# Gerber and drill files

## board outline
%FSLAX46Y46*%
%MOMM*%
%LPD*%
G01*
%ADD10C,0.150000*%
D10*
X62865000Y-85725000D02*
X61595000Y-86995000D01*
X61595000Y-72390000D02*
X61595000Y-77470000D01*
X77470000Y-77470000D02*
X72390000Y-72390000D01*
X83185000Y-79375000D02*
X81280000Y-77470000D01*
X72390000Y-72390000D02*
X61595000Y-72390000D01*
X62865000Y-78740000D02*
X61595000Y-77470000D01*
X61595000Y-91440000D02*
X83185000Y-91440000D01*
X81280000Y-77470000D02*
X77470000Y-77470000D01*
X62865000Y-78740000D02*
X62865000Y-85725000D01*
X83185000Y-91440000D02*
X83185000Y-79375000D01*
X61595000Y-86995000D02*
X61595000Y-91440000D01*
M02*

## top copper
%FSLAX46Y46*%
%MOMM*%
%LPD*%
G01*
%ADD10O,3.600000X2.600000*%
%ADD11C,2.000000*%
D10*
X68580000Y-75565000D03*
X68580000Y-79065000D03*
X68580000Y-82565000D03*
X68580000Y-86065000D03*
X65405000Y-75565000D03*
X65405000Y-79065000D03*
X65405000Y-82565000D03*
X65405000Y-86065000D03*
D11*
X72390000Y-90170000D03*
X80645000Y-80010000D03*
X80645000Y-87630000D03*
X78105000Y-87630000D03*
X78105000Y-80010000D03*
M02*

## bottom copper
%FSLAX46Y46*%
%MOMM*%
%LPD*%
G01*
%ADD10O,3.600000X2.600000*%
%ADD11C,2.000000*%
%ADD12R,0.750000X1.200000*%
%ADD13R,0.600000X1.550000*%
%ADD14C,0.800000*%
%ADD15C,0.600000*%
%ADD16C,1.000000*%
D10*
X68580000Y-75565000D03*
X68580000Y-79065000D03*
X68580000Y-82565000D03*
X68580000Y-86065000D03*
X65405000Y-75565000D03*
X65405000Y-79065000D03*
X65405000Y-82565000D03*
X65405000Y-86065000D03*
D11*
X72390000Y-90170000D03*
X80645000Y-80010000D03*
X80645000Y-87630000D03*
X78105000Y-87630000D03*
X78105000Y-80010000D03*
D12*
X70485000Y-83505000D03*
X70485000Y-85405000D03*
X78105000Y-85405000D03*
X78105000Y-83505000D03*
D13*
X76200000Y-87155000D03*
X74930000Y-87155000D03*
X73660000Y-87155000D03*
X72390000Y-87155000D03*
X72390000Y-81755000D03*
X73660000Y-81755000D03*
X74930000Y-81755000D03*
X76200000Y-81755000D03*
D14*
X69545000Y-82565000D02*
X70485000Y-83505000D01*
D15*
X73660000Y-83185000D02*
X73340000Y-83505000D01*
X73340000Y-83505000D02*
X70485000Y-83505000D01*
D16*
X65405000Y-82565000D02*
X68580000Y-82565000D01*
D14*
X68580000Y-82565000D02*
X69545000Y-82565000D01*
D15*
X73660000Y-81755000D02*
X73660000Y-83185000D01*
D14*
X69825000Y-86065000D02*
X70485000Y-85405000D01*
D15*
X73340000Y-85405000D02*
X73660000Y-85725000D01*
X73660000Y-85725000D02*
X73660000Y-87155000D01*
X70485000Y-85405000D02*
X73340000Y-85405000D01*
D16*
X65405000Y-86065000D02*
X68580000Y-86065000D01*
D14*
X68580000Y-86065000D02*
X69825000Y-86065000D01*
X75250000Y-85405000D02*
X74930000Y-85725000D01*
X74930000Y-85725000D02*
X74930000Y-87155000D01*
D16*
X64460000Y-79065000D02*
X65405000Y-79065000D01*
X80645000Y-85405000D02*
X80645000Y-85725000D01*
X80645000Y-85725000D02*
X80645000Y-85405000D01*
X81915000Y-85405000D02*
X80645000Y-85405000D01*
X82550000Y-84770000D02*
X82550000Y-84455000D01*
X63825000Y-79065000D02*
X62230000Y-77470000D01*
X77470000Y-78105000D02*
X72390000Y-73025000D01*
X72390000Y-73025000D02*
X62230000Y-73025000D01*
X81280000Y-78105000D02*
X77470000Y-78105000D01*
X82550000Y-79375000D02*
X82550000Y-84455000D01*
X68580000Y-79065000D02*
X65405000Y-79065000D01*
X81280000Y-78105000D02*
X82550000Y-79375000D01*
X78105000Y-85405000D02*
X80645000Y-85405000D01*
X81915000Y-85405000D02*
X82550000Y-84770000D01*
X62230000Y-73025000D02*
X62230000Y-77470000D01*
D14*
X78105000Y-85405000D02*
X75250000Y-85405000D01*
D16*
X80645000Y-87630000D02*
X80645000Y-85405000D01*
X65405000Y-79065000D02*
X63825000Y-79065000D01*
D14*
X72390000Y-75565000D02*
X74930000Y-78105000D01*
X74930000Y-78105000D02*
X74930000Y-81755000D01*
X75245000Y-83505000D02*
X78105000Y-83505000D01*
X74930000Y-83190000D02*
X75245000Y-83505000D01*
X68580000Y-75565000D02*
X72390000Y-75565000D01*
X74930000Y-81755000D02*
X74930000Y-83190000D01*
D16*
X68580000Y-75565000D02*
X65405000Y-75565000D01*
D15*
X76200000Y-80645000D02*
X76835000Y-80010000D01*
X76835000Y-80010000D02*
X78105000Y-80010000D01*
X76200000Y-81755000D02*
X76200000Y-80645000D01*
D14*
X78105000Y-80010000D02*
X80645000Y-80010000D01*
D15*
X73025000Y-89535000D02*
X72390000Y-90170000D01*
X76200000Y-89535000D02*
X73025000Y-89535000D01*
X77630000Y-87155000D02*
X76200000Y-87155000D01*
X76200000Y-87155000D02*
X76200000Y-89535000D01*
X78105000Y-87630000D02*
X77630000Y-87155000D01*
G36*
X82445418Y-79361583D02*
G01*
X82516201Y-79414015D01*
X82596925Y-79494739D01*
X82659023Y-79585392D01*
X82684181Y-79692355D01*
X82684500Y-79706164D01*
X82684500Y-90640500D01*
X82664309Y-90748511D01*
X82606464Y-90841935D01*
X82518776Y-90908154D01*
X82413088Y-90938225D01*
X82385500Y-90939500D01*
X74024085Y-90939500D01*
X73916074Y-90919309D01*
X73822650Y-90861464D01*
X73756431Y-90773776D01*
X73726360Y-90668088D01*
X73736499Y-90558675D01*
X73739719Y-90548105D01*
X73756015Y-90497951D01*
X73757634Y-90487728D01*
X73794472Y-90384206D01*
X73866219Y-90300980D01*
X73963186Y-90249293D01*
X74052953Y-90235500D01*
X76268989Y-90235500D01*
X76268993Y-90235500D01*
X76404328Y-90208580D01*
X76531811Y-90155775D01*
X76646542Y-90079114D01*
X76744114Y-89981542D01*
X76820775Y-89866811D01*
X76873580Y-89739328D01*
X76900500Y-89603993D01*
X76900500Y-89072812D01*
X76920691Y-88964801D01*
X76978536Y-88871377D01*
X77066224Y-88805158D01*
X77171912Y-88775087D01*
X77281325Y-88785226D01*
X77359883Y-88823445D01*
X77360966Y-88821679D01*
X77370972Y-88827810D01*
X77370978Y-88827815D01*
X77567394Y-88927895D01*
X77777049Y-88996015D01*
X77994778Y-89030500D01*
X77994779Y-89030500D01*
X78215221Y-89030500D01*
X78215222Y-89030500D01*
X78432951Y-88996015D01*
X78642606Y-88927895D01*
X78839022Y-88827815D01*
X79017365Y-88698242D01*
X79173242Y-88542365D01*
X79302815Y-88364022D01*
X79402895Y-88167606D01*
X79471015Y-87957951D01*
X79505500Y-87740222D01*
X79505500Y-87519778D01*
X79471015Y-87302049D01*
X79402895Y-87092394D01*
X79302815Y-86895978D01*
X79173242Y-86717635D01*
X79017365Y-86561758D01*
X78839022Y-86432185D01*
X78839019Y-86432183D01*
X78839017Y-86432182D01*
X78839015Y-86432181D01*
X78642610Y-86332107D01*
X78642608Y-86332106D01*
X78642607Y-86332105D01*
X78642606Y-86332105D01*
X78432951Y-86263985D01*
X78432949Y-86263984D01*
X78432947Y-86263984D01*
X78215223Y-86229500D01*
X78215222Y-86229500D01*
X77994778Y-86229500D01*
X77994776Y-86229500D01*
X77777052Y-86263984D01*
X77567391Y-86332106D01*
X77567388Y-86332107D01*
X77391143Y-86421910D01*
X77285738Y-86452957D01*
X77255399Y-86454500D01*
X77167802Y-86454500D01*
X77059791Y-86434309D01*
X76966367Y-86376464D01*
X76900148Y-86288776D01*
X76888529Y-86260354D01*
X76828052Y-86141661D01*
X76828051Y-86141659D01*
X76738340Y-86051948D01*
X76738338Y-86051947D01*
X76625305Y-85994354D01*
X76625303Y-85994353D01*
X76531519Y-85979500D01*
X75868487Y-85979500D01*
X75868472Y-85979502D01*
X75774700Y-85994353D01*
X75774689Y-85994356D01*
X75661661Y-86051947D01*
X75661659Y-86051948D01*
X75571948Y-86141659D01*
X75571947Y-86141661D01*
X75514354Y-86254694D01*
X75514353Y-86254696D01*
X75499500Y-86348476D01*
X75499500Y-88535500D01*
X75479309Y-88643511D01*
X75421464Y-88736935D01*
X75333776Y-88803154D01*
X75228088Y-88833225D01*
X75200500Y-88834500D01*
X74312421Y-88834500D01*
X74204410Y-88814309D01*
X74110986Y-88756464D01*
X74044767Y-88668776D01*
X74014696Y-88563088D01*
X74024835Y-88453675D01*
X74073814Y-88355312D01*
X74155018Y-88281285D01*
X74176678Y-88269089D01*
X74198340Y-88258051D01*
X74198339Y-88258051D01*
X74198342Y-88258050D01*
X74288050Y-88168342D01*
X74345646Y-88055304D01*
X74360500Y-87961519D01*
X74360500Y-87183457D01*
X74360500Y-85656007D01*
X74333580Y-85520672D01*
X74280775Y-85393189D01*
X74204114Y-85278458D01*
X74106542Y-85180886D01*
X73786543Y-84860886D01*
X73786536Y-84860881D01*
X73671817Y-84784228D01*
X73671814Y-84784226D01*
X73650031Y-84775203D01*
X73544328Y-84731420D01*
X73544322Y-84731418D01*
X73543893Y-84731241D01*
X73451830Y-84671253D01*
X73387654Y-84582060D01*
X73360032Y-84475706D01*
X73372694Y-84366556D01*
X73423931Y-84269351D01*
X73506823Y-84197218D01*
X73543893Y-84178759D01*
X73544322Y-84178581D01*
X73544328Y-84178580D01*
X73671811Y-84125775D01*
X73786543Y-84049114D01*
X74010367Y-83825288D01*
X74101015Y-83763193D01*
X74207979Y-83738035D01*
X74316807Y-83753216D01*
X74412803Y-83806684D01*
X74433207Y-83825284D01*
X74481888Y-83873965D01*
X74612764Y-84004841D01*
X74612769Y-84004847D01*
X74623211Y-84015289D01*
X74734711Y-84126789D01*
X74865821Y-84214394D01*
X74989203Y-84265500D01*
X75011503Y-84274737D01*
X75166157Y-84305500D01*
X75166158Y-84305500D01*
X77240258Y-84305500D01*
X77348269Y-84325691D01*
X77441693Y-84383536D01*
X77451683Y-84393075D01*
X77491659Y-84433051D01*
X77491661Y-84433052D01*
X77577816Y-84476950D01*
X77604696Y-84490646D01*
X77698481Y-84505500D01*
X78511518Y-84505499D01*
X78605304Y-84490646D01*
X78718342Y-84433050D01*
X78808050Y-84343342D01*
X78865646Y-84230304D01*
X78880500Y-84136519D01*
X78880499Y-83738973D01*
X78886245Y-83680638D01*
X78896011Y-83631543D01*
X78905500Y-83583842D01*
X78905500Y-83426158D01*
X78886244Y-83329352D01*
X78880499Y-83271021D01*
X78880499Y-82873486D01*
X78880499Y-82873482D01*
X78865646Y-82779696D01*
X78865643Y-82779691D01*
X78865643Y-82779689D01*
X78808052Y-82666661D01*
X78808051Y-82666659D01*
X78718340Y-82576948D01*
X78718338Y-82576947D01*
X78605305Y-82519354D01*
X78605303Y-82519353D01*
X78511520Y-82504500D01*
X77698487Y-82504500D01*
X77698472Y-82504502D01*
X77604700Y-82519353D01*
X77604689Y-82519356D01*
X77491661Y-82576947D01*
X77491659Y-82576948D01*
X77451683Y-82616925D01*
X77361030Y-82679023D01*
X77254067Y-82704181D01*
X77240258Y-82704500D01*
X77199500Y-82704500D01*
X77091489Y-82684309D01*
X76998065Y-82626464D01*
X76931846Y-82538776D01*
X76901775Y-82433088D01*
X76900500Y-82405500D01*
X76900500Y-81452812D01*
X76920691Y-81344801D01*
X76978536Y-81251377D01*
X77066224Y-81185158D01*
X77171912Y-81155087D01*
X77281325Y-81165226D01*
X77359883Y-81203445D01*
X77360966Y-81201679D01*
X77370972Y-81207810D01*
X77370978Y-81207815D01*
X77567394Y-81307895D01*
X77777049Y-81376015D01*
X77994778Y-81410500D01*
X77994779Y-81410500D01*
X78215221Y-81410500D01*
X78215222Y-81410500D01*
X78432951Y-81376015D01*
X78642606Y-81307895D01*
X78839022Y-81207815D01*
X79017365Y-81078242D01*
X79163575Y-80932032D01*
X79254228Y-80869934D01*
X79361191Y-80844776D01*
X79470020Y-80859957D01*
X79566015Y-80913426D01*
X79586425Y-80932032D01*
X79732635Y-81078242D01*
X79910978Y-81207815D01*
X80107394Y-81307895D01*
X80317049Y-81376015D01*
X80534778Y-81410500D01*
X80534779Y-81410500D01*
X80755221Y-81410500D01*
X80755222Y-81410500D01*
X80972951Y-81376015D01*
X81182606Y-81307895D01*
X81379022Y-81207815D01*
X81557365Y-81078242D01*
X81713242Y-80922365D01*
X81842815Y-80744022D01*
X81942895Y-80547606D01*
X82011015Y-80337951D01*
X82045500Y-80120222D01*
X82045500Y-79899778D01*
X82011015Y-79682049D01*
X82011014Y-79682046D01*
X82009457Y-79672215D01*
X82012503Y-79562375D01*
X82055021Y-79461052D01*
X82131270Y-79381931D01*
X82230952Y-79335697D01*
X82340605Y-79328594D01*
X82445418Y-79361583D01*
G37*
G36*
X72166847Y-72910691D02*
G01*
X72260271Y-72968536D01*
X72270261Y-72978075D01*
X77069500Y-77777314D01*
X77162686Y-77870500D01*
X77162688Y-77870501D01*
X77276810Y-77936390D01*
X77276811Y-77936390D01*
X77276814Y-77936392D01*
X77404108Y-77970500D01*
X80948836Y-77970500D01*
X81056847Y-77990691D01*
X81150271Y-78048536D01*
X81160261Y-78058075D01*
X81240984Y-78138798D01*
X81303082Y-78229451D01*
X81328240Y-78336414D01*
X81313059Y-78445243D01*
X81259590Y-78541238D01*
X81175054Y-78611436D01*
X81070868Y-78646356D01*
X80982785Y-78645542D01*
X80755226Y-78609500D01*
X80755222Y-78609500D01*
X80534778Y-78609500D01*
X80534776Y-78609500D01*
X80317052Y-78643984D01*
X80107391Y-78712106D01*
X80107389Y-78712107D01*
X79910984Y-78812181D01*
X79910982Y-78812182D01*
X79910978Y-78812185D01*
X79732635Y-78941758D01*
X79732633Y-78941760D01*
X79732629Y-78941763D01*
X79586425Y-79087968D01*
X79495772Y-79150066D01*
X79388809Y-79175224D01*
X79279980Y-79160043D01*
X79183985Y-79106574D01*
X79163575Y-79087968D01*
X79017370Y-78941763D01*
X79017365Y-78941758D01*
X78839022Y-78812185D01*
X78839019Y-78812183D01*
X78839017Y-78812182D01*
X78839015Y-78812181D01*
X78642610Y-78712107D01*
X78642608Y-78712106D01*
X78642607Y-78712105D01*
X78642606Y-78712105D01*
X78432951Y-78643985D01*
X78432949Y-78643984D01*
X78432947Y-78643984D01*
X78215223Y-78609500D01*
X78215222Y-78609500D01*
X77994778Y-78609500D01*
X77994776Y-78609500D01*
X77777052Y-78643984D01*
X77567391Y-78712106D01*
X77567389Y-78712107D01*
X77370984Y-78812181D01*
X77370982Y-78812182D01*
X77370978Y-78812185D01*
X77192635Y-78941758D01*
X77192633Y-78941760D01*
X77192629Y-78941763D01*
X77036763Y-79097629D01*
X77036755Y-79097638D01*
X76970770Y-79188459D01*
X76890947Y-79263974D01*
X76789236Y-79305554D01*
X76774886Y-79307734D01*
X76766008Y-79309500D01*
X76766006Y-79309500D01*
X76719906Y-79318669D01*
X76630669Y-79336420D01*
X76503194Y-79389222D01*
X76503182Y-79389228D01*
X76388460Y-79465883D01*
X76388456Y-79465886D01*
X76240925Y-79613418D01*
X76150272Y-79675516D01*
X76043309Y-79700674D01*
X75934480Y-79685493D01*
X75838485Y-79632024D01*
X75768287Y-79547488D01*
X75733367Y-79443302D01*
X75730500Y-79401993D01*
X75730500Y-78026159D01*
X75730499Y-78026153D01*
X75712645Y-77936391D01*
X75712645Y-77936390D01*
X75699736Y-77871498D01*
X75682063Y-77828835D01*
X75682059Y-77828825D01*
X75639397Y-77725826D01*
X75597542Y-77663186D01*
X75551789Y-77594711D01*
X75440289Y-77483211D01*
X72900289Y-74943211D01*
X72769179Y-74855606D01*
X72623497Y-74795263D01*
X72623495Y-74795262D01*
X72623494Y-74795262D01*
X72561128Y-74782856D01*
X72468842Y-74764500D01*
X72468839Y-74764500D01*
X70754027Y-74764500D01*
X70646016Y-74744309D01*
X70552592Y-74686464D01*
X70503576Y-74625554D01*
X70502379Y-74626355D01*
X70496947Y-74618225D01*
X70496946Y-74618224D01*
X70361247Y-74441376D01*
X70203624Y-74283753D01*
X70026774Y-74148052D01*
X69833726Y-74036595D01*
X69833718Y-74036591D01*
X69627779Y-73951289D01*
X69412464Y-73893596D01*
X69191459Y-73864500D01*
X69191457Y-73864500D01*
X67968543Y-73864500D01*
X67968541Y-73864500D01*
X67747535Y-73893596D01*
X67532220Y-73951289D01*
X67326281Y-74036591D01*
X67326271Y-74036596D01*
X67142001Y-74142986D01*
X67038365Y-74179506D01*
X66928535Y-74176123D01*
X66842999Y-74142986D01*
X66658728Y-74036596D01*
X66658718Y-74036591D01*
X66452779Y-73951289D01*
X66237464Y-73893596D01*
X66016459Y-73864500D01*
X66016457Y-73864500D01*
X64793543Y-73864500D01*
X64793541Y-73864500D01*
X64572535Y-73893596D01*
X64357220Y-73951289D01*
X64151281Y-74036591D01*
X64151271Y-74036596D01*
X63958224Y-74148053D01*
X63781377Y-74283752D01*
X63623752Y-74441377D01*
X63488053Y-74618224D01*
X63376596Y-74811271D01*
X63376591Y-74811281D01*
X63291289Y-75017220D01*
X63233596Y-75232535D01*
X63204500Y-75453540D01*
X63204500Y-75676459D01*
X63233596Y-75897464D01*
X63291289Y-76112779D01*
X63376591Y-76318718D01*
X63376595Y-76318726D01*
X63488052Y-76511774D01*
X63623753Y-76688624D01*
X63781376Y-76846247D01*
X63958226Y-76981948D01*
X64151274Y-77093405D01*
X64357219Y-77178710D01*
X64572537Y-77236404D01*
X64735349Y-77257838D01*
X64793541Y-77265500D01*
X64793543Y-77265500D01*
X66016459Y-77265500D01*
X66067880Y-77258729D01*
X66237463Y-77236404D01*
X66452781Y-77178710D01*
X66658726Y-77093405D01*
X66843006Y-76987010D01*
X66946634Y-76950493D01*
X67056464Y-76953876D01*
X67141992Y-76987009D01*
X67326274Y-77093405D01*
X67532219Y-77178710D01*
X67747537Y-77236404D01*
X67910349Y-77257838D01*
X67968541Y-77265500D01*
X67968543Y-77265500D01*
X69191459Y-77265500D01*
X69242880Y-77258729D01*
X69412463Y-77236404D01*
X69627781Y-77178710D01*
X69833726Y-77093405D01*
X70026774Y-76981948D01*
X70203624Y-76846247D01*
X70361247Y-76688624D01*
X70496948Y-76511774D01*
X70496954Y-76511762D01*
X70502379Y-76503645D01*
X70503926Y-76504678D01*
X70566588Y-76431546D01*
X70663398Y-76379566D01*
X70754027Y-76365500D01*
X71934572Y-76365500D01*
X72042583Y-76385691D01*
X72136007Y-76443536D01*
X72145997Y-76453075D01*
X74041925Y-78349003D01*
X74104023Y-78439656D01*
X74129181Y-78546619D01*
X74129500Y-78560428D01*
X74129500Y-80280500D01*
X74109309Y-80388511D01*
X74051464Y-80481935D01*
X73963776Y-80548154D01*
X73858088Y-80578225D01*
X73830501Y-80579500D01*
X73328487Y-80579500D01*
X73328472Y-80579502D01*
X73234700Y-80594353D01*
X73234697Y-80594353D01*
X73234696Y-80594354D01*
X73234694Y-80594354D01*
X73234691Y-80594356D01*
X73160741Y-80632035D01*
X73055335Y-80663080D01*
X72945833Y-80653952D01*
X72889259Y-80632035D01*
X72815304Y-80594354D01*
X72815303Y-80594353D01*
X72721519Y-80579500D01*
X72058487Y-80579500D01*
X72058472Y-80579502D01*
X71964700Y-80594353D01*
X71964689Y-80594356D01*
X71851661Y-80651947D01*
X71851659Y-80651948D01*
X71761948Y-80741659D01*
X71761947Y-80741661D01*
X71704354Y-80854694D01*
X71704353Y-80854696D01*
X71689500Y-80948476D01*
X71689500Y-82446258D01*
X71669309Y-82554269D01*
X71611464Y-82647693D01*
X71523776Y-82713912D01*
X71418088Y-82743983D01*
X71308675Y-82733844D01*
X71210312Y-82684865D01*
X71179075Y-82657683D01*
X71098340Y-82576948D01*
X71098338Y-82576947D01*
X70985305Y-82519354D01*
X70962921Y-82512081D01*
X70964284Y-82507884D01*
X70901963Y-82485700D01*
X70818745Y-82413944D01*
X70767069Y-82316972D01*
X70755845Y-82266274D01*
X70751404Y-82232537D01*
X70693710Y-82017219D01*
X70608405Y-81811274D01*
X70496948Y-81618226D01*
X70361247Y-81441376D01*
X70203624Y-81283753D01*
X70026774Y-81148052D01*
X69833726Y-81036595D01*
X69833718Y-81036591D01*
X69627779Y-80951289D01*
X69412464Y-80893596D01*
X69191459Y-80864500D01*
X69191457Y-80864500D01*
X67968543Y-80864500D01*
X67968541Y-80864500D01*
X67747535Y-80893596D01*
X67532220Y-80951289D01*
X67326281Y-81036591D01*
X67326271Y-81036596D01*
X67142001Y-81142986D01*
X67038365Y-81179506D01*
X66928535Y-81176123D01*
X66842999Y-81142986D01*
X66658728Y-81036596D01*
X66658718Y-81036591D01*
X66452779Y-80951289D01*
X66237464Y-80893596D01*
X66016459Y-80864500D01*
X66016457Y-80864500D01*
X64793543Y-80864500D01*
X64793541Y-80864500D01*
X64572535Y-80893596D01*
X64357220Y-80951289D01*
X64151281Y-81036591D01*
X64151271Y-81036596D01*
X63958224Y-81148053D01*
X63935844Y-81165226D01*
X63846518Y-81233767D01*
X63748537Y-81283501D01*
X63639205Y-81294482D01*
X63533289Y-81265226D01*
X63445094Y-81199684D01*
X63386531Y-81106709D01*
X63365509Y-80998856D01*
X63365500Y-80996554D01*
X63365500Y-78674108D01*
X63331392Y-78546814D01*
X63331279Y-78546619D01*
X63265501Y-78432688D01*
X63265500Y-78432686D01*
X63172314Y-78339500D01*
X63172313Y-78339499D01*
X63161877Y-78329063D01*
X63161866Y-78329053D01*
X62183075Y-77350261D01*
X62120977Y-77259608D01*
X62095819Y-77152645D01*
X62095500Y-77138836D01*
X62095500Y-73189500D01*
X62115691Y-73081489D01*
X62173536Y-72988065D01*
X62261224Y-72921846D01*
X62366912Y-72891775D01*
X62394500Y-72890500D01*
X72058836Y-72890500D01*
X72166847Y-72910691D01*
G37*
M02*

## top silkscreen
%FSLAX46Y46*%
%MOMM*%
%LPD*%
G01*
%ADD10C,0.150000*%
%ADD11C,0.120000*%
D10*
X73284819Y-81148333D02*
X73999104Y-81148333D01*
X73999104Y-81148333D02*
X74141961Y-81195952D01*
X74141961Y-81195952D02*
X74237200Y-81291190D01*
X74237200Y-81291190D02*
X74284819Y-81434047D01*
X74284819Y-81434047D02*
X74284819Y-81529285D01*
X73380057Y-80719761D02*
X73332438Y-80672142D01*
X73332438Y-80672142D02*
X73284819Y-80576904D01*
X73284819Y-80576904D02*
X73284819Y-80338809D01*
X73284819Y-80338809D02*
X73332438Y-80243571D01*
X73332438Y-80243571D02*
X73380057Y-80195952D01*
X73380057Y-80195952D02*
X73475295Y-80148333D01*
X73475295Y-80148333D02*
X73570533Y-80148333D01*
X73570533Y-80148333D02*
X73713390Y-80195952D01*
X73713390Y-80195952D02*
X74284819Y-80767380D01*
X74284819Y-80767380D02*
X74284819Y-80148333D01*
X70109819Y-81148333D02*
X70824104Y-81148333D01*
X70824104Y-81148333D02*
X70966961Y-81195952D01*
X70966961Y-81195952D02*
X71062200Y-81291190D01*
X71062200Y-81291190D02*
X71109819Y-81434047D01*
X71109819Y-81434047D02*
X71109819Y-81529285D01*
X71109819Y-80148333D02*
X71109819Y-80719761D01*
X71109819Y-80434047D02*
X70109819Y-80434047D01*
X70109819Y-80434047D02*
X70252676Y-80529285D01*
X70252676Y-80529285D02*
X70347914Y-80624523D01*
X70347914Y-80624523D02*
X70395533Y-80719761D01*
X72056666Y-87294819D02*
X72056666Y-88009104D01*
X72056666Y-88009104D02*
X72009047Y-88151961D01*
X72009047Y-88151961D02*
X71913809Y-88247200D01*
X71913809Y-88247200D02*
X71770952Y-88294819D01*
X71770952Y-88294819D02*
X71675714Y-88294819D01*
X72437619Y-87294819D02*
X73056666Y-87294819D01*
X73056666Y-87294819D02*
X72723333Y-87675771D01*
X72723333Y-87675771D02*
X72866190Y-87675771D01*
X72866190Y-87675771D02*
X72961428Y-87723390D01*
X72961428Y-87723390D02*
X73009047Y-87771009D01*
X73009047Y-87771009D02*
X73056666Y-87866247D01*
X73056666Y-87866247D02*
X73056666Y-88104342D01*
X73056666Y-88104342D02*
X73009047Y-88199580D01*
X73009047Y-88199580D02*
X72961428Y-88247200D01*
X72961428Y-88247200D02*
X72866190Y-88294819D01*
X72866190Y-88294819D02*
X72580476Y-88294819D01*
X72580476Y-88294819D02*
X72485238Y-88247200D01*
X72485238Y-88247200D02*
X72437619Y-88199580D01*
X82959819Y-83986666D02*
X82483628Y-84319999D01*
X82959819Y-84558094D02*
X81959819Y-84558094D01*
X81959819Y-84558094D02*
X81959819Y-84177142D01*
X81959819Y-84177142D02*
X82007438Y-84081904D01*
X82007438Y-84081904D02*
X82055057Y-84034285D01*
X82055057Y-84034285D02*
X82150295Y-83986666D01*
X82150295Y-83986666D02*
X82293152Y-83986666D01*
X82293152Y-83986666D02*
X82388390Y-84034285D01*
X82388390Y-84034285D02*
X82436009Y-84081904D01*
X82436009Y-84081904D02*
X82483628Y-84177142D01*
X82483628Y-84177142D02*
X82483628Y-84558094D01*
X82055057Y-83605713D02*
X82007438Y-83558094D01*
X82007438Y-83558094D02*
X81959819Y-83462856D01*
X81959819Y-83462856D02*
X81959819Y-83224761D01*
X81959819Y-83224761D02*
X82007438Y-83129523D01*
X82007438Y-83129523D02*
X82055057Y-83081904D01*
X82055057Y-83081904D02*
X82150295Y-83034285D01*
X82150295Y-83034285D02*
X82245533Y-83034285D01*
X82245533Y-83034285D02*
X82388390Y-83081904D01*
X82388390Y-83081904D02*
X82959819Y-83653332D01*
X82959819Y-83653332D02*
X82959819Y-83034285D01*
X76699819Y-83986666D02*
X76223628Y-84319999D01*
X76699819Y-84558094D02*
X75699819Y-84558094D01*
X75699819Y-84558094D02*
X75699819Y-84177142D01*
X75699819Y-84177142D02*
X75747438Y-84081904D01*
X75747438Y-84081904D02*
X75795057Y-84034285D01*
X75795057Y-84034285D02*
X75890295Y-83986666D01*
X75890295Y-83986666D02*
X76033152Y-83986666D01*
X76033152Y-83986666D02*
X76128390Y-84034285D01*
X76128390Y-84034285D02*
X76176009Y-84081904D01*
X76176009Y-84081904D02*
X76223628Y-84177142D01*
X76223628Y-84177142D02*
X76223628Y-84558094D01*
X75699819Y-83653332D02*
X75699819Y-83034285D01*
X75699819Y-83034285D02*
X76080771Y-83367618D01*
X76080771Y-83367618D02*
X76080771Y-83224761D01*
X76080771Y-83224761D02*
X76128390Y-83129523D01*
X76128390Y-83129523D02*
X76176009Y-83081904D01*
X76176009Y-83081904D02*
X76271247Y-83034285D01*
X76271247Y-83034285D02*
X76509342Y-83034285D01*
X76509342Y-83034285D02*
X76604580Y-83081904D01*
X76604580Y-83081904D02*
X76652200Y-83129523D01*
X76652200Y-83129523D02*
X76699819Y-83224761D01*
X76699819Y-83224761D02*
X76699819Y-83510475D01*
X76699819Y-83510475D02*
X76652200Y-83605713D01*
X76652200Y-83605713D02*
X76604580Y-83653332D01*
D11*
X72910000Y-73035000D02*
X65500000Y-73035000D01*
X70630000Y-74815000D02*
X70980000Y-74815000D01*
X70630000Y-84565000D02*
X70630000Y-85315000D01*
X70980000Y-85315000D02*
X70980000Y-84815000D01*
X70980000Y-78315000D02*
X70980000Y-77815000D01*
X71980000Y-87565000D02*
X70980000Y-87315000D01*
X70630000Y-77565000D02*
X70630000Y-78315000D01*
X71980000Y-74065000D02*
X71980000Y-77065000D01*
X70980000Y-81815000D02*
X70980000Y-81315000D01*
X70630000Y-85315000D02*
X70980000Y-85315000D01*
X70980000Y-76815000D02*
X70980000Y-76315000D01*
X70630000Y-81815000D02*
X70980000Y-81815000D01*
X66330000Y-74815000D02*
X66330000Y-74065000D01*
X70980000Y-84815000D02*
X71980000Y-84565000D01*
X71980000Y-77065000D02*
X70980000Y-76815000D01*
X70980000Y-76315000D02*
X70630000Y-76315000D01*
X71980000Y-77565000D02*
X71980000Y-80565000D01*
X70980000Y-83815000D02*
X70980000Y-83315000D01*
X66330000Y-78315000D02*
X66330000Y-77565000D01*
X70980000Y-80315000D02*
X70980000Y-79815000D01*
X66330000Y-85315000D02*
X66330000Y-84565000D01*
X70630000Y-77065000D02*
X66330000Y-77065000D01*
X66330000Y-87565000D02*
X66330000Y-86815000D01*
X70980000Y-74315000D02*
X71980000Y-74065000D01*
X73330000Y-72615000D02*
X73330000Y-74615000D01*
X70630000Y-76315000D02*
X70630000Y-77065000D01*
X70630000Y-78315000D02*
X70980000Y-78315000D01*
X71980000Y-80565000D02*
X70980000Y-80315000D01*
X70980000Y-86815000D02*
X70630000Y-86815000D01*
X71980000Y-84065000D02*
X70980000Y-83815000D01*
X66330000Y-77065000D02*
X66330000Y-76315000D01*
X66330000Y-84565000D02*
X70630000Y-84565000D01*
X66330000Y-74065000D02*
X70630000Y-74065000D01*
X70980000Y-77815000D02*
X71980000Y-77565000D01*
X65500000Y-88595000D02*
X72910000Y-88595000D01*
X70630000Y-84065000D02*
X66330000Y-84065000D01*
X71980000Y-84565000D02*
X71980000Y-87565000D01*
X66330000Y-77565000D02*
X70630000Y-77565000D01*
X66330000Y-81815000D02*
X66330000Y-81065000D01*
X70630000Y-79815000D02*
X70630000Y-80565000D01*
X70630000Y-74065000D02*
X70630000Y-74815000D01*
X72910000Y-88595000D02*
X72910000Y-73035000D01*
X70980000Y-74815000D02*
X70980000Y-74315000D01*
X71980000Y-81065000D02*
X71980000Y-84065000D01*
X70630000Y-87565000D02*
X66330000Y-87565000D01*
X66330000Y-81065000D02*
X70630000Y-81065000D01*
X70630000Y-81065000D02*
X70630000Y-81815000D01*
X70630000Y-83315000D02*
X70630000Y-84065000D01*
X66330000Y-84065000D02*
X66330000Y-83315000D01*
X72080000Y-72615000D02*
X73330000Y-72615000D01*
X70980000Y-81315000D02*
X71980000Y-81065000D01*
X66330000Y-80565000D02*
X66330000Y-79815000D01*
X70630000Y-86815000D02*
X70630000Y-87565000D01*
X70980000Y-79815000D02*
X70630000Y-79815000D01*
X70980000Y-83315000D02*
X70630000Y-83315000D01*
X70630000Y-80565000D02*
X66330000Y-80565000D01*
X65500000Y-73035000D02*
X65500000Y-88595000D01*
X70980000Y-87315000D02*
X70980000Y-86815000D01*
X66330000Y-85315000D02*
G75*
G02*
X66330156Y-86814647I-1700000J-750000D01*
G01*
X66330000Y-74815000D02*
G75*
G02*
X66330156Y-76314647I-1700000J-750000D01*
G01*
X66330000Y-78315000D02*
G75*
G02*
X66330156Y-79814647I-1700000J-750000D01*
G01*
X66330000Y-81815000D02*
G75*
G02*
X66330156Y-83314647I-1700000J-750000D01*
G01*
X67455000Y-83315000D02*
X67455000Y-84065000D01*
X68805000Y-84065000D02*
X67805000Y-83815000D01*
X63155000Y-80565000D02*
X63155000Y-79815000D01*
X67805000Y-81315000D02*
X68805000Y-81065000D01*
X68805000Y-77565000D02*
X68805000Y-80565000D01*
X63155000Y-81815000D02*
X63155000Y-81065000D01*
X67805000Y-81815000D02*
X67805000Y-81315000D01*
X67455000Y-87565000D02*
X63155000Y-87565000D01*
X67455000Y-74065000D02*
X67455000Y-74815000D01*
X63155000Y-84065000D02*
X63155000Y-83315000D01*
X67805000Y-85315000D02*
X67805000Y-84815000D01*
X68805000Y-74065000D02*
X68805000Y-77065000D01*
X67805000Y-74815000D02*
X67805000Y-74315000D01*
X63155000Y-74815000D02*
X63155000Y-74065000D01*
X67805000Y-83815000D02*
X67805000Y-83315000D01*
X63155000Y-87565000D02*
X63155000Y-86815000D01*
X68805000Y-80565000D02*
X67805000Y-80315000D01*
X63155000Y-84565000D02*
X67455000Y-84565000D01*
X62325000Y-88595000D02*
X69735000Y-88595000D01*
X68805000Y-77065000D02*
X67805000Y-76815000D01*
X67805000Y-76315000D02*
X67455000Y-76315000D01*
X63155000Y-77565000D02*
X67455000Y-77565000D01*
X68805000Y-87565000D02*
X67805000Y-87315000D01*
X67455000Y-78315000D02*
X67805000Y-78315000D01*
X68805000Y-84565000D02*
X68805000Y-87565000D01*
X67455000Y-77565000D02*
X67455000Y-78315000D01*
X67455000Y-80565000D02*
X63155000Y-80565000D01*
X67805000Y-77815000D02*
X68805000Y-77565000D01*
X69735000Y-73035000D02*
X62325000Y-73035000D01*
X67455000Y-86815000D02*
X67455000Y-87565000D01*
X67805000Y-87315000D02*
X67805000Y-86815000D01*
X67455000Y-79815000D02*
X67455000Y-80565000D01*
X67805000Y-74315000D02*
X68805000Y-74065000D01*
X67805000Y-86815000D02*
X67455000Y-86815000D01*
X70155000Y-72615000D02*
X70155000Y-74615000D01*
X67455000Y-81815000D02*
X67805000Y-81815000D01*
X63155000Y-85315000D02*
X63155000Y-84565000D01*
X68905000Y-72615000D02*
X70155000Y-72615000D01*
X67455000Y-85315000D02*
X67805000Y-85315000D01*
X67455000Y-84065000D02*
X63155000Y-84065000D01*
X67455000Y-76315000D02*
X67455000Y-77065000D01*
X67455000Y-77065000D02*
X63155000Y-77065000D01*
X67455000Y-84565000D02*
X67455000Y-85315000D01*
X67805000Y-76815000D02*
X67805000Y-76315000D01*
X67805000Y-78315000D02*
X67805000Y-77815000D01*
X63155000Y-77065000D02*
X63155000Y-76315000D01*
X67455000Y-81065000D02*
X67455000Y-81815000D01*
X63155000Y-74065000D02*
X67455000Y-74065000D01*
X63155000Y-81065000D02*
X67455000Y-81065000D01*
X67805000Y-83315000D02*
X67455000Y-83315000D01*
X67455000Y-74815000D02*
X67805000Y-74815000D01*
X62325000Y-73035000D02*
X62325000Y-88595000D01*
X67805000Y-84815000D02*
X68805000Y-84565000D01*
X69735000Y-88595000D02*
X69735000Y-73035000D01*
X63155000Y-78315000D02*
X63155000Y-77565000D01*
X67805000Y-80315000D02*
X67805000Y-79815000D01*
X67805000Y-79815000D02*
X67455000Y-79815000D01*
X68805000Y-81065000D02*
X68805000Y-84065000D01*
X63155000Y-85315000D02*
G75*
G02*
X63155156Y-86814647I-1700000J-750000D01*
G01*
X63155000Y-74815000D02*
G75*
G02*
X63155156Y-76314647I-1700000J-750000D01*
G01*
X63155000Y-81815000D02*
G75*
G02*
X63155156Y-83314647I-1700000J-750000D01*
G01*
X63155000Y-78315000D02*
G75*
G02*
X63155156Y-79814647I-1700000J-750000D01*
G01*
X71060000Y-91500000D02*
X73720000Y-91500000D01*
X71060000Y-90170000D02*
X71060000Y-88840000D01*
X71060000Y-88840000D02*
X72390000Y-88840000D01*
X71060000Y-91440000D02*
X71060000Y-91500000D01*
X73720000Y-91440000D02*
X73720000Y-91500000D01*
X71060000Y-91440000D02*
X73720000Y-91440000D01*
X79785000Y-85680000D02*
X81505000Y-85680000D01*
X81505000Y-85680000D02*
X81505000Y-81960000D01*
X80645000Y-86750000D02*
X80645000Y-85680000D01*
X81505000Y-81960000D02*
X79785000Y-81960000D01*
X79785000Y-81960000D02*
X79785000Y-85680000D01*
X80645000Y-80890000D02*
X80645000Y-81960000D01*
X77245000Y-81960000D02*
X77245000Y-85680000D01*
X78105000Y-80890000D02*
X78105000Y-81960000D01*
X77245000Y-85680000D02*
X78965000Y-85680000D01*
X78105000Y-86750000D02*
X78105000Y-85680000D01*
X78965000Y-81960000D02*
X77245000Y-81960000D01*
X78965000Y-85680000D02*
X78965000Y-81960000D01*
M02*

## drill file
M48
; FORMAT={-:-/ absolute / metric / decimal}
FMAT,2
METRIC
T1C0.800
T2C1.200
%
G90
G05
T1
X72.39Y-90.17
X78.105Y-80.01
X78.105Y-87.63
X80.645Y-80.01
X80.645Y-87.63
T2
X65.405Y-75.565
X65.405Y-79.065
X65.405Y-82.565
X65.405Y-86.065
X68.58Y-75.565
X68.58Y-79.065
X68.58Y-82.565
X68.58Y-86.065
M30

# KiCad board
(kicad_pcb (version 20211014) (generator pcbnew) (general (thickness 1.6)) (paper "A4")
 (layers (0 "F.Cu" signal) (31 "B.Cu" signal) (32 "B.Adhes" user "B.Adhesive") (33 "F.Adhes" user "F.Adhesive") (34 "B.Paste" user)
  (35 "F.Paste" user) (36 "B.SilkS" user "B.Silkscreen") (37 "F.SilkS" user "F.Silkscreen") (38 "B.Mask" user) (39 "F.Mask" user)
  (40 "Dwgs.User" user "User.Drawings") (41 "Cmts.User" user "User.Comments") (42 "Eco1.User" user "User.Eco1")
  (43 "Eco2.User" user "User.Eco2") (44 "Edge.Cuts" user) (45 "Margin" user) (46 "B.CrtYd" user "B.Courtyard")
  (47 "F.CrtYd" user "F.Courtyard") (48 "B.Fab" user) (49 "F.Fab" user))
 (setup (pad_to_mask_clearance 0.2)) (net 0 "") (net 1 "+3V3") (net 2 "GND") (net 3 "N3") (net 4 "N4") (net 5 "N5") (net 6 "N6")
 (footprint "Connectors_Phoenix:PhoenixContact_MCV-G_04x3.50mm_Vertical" (layer "F.Cu") (at 68.58 75.565 -90)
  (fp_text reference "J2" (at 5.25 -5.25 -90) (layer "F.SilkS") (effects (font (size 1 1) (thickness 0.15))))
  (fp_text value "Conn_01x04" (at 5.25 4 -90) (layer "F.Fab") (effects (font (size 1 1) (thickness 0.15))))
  (fp_line (start -2.53 -4.33) (end -2.53 3.08) (layer "F.SilkS") (width 0.12))
  (fp_line (start -0.75 -2.05) (end -0.75 -2.4) (layer "F.SilkS") (width 0.12))
  (fp_line (start 9 -2.05) (end 9.75 -2.05) (layer "F.SilkS") (width 0.12))
  (fp_line (start 9.75 -2.4) (end 9.25 -2.4) (layer "F.SilkS") (width 0.12))
  (fp_line (start 2.75 -2.4) (end 2.25 -2.4) (layer "F.SilkS") (width 0.12))
  (fp_line (start 12 -3.4) (end 11.75 -2.4) (layer "F.SilkS") (width 0.12))
  (fp_line (start 2 -2.05) (end 2.75 -2.05) (layer "F.SilkS") (width 0.12))
  (fp_line (start -1.5 -3.4) (end 1.5 -3.4) (layer "F.SilkS") (width 0.12))
  (fp_line (start 6.25 -2.4) (end 5.75 -2.4) (layer "F.SilkS") (width 0.12))
  (fp_line (start 9.75 -2.05) (end 9.75 -2.4) (layer "F.SilkS") (width 0.12))
  (fp_line (start 1.25 -2.4) (end 0.75 -2.4) (layer "F.SilkS") (width 0.12))
  (fp_line (start 6.25 -2.05) (end 6.25 -2.4) (layer "F.SilkS") (width 0.12))
  (fp_line (start -0.75 2.25) (end -1.5 2.25) (layer "F.SilkS") (width 0.12))
  (fp_line (start 9.25 -2.4) (end 9 -3.4) (layer "F.SilkS") (width 0.12))
  (fp_line (start 1.5 -3.4) (end 1.25 -2.4) (layer "F.SilkS") (width 0.12))
  (fp_line (start 0.75 -2.4) (end 0.75 -2.05) (layer "F.SilkS") (width 0.12))
  (fp_line (start 2 -3.4) (end 5 -3.4) (layer "F.SilkS") (width 0.12))
  (fp_line (start 8.25 -2.4) (end 7.75 -2.4) (layer "F.SilkS") (width 0.12))
  (fp_line (start 2.75 2.25) (end 2 2.25) (layer "F.SilkS") (width 0.12))
  (fp_line (start 4.75 -2.4) (end 4.25 -2.4) (layer "F.SilkS") (width 0.12))
  (fp_line (start 9.75 2.25) (end 9 2.25) (layer "F.SilkS") (width 0.12))
  (fp_line (start 1.5 -2.05) (end 1.5 2.25) (layer "F.SilkS") (width 0.12))
  (fp_line (start 12 2.25) (end 11.25 2.25) (layer "F.SilkS") (width 0.12))
  (fp_line (start -1.25 -2.4) (end -1.5 -3.4) (layer "F.SilkS") (width 0.12))
  (fp_line (start -2.95 -4.75) (end -0.95 -4.75) (layer "F.SilkS") (width 0.12))
  (fp_line (start 0.75 -2.05) (end 1.5 -2.05) (layer "F.SilkS") (width 0.12))
  (fp_line (start 2.75 -2.05) (end 2.75 -2.4) (layer "F.SilkS") (width 0.12))
  (fp_line (start 5 -3.4) (end 4.75 -2.4) (layer "F.SilkS") (width 0.12))
  (fp_line (start 11.25 -2.4) (end 11.25 -2.05) (layer "F.SilkS") (width 0.12))
  (fp_line (start 8.5 -3.4) (end 8.25 -2.4) (layer "F.SilkS") (width 0.12))
  (fp_line (start 1.5 2.25) (end 0.75 2.25) (layer "F.SilkS") (width 0.12))
  (fp_line (start 9 2.25) (end 9 -2.05) (layer "F.SilkS") (width 0.12))
  (fp_line (start -1.5 2.25) (end -1.5 -2.05) (layer "F.SilkS") (width 0.12))
  (fp_line (start 2.25 -2.4) (end 2 -3.4) (layer "F.SilkS") (width 0.12))
  (fp_line (start 13.03 3.08) (end 13.03 -4.33) (layer "F.SilkS") (width 0.12))
  (fp_line (start 8.5 -2.05) (end 8.5 2.25) (layer "F.SilkS") (width 0.12))
  (fp_line (start 9 -3.4) (end 12 -3.4) (layer "F.SilkS") (width 0.12))
  (fp_line (start 2 2.25) (end 2 -2.05) (layer "F.SilkS") (width 0.12))
  (fp_line (start 6.25 2.25) (end 5.5 2.25) (layer "F.SilkS") (width 0.12))
  (fp_line (start 4.25 -2.05) (end 5 -2.05) (layer "F.SilkS") (width 0.12))
  (fp_line (start -1.5 -2.05) (end -0.75 -2.05) (layer "F.SilkS") (width 0.12))
  (fp_line (start 13.03 -4.33) (end -2.53 -4.33) (layer "F.SilkS") (width 0.12))
  (fp_line (start -0.75 -2.4) (end -1.25 -2.4) (layer "F.SilkS") (width 0.12))
  (fp_line (start 5.5 -3.4) (end 8.5 -3.4) (layer "F.SilkS") (width 0.12))
  (fp_line (start 12 -2.05) (end 12 2.25) (layer "F.SilkS") (width 0.12))
  (fp_line (start 5.5 2.25) (end 5.5 -2.05) (layer "F.SilkS") (width 0.12))
  (fp_line (start 5.5 -2.05) (end 6.25 -2.05) (layer "F.SilkS") (width 0.12))
  (fp_line (start 7.75 -2.05) (end 8.5 -2.05) (layer "F.SilkS") (width 0.12))
  (fp_line (start 8.5 2.25) (end 7.75 2.25) (layer "F.SilkS") (width 0.12))
  (fp_line (start -2.95 -3.5) (end -2.95 -4.75) (layer "F.SilkS") (width 0.12))
  (fp_line (start 5.75 -2.4) (end 5.5 -3.4) (layer "F.SilkS") (width 0.12))
  (fp_line (start 5 2.25) (end 4.25 2.25) (layer "F.SilkS") (width 0.12))
  (fp_line (start 11.25 -2.05) (end 12 -2.05) (layer "F.SilkS") (width 0.12))
  (fp_line (start 4.25 -2.4) (end 4.25 -2.05) (layer "F.SilkS") (width 0.12))
  (fp_line (start 7.75 -2.4) (end 7.75 -2.05) (layer "F.SilkS") (width 0.12))
  (fp_line (start 5 -2.05) (end 5 2.25) (layer "F.SilkS") (width 0.12))
  (fp_line (start -2.53 3.08) (end 13.03 3.08) (layer "F.SilkS") (width 0.12))
  (fp_line (start 11.75 -2.4) (end 11.25 -2.4) (layer "F.SilkS") (width 0.12))
  (fp_arc (start 9.75 2.25) (mid 10.499807 2.09191) (end 11.249647 2.249844) (layer "F.SilkS") (width 0.12))
  (fp_arc (start -0.75 2.25) (mid -0.000193 2.09191) (end 0.749647 2.249844) (layer "F.SilkS") (width 0.12))
  (fp_arc (start 2.75 2.25) (mid 3.499807 2.09191) (end 4.249647 2.249844) (layer "F.SilkS") (width 0.12))
  (fp_arc (start 6.25 2.25) (mid 6.999807 2.09191) (end 7.749647 2.249844) (layer "F.SilkS") (width 0.12))
  (pad "1" thru_hole oval locked (at 0 0 270) (size 2.6 3.6) (drill 1.2) (layers *.Cu *.Mask) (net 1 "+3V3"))
  (pad "2" thru_hole oval locked (at 3.5 0 270) (size 2.6 3.6) (drill 1.2) (layers *.Cu *.Mask) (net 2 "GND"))
  (pad "3" thru_hole oval locked (at 7 0 270) (size 2.6 3.6) (drill 1.2) (layers *.Cu *.Mask) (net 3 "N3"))
  (pad "4" thru_hole oval locked (at 10.5 0 270) (size 2.6 3.6) (drill 1.2) (layers *.Cu *.Mask) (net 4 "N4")))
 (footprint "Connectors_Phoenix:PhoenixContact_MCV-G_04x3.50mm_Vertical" (layer "F.Cu") (at 65.405 75.565 -90)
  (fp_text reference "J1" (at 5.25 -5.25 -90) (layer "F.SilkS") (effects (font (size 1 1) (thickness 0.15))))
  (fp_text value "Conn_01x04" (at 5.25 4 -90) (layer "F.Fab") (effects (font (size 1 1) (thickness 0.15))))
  (fp_line (start 7.75 -2.05) (end 8.5 -2.05) (layer "F.SilkS") (width 0.12))
  (fp_line (start 8.5 -3.4) (end 8.25 -2.4) (layer "F.SilkS") (width 0.12))
  (fp_line (start 5 2.25) (end 4.25 2.25) (layer "F.SilkS") (width 0.12))
  (fp_line (start 5.75 -2.4) (end 5.5 -3.4) (layer "F.SilkS") (width 0.12))
  (fp_line (start 2 -3.4) (end 5 -3.4) (layer "F.SilkS") (width 0.12))
  (fp_line (start 6.25 2.25) (end 5.5 2.25) (layer "F.SilkS") (width 0.12))
  (fp_line (start 6.25 -2.4) (end 5.75 -2.4) (layer "F.SilkS") (width 0.12))
  (fp_line (start 12 -2.05) (end 12 2.25) (layer "F.SilkS") (width 0.12))
  (fp_line (start -1.5 -2.05) (end -0.75 -2.05) (layer "F.SilkS") (width 0.12))
  (fp_line (start 8.5 2.25) (end 7.75 2.25) (layer "F.SilkS") (width 0.12))
  (fp_line (start 9.75 -2.4) (end 9.25 -2.4) (layer "F.SilkS") (width 0.12))
  (fp_line (start -1.5 -3.4) (end 1.5 -3.4) (layer "F.SilkS") (width 0.12))
  (fp_line (start -0.75 -2.4) (end -1.25 -2.4) (layer "F.SilkS") (width 0.12))
  (fp_line (start -0.75 2.25) (end -1.5 2.25) (layer "F.SilkS") (width 0.12))
  (fp_line (start 8.25 -2.4) (end 7.75 -2.4) (layer "F.SilkS") (width 0.12))
  (fp_line (start 12 2.25) (end 11.25 2.25) (layer "F.SilkS") (width 0.12))
  (fp_line (start 5 -3.4) (end 4.75 -2.4) (layer "F.SilkS") (width 0.12))
  (fp_line (start 9 2.25) (end 9 -2.05) (layer "F.SilkS") (width 0.12))
  (fp_line (start 13.03 3.08) (end 13.03 -4.33) (layer "F.SilkS") (width 0.12))
  (fp_line (start 1.5 -3.4) (end 1.25 -2.4) (layer "F.SilkS") (width 0.12))
  (fp_line (start 0.75 -2.4) (end 0.75 -2.05) (layer "F.SilkS") (width 0.12))
  (fp_line (start 2 2.25) (end 2 -2.05) (layer "F.SilkS") (width 0.12))
  (fp_line (start 12 -3.4) (end 11.75 -2.4) (layer "F.SilkS") (width 0.12))
  (fp_line (start 2.75 -2.05) (end 2.75 -2.4) (layer "F.SilkS") (width 0.12))
  (fp_line (start 9 -3.4) (end 12 -3.4) (layer "F.SilkS") (width 0.12))
  (fp_line (start 2 -2.05) (end 2.75 -2.05) (layer "F.SilkS") (width 0.12))
  (fp_line (start 5 -2.05) (end 5 2.25) (layer "F.SilkS") (width 0.12))
  (fp_line (start 2.25 -2.4) (end 2 -3.4) (layer "F.SilkS") (width 0.12))
  (fp_line (start -2.53 -4.33) (end -2.53 3.08) (layer "F.SilkS") (width 0.12))
  (fp_line (start 11.25 -2.05) (end 12 -2.05) (layer "F.SilkS") (width 0.12))
  (fp_line (start 11.75 -2.4) (end 11.25 -2.4) (layer "F.SilkS") (width 0.12))
  (fp_line (start 4.25 -2.05) (end 5 -2.05) (layer "F.SilkS") (width 0.12))
  (fp_line (start -1.25 -2.4) (end -1.5 -3.4) (layer "F.SilkS") (width 0.12))
  (fp_line (start 11.25 -2.4) (end 11.25 -2.05) (layer "F.SilkS") (width 0.12))
  (fp_line (start -2.95 -4.75) (end -0.95 -4.75) (layer "F.SilkS") (width 0.12))
  (fp_line (start 6.25 -2.05) (end 6.25 -2.4) (layer "F.SilkS") (width 0.12))
  (fp_line (start 9.75 2.25) (end 9 2.25) (layer "F.SilkS") (width 0.12))
  (fp_line (start -2.95 -3.5) (end -2.95 -4.75) (layer "F.SilkS") (width 0.12))
  (fp_line (start 9.75 -2.05) (end 9.75 -2.4) (layer "F.SilkS") (width 0.12))
  (fp_line (start 8.5 -2.05) (end 8.5 2.25) (layer "F.SilkS") (width 0.12))
  (fp_line (start 0.75 -2.05) (end 1.5 -2.05) (layer "F.SilkS") (width 0.12))
  (fp_line (start 1.5 -2.05) (end 1.5 2.25) (layer "F.SilkS") (width 0.12))
  (fp_line (start 9 -2.05) (end 9.75 -2.05) (layer "F.SilkS") (width 0.12))
  (fp_line (start 1.25 -2.4) (end 0.75 -2.4) (layer "F.SilkS") (width 0.12))
  (fp_line (start 2.75 -2.4) (end 2.25 -2.4) (layer "F.SilkS") (width 0.12))
  (fp_line (start 1.5 2.25) (end 0.75 2.25) (layer "F.SilkS") (width 0.12))
  (fp_line (start 5.5 -2.05) (end 6.25 -2.05) (layer "F.SilkS") (width 0.12))
  (fp_line (start -1.5 2.25) (end -1.5 -2.05) (layer "F.SilkS") (width 0.12))
  (fp_line (start 5.5 2.25) (end 5.5 -2.05) (layer "F.SilkS") (width 0.12))
  (fp_line (start 7.75 -2.4) (end 7.75 -2.05) (layer "F.SilkS") (width 0.12))
  (fp_line (start -0.75 -2.05) (end -0.75 -2.4) (layer "F.SilkS") (width 0.12))
  (fp_line (start -2.53 3.08) (end 13.03 3.08) (layer "F.SilkS") (width 0.12))
  (fp_line (start 9.25 -2.4) (end 9 -3.4) (layer "F.SilkS") (width 0.12))
  (fp_line (start 13.03 -4.33) (end -2.53 -4.33) (layer "F.SilkS") (width 0.12))
  (fp_line (start 2.75 2.25) (end 2 2.25) (layer "F.SilkS") (width 0.12))
  (fp_line (start 4.75 -2.4) (end 4.25 -2.4) (layer "F.SilkS") (width 0.12))
  (fp_line (start 4.25 -2.4) (end 4.25 -2.05) (layer "F.SilkS") (width 0.12))
  (fp_line (start 5.5 -3.4) (end 8.5 -3.4) (layer "F.SilkS") (width 0.12))
  (fp_arc (start 9.75 2.25) (mid 10.499807 2.09191) (end 11.249647 2.249844) (layer "F.SilkS") (width 0.12))
  (fp_arc (start -0.75 2.25) (mid -0.000193 2.09191) (end 0.749647 2.249844) (layer "F.SilkS") (width 0.12))
  (fp_arc (start 6.25 2.25) (mid 6.999807 2.09191) (end 7.749647 2.249844) (layer "F.SilkS") (width 0.12))
  (fp_arc (start 2.75 2.25) (mid 3.499807 2.09191) (end 4.249647 2.249844) (layer "F.SilkS") (width 0.12))
  (pad "1" thru_hole oval locked (at 0 0 270) (size 2.6 3.6) (drill 1.2) (layers *.Cu *.Mask) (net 1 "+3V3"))
  (pad "2" thru_hole oval locked (at 3.5 0 270) (size 2.6 3.6) (drill 1.2) (layers *.Cu *.Mask) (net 2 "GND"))
  (pad "3" thru_hole oval locked (at 7 0 270) (size 2.6 3.6) (drill 1.2) (layers *.Cu *.Mask) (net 3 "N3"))
  (pad "4" thru_hole oval locked (at 10.5 0 270) (size 2.6 3.6) (drill 1.2) (layers *.Cu *.Mask) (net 4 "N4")))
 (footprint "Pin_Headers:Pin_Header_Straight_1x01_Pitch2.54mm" (layer "F.Cu") (at 72.39 90.17)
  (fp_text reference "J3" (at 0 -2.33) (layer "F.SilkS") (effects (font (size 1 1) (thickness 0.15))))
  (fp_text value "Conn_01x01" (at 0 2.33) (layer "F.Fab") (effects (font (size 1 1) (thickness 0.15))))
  (fp_line (start -1.33 1.33) (end 1.33 1.33) (layer "F.SilkS") (width 0.12))
  (fp_line (start -1.33 0) (end -1.33 -1.33) (layer "F.SilkS") (width 0.12))
  (fp_line (start -1.33 -1.33) (end 0 -1.33) (layer "F.SilkS") (width 0.12))
  (fp_line (start -1.33 1.27) (end -1.33 1.33) (layer "F.SilkS") (width 0.12))
  (fp_line (start 1.33 1.27) (end 1.33 1.33) (layer "F.SilkS") (width 0.12))
  (fp_line (start -1.33 1.27) (end 1.33 1.27) (layer "F.SilkS") (width 0.12))
  (pad "1" thru_hole circle locked (at 0 0) (size 2 2) (drill 0.8) (layers *.Cu *.Mask) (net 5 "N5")))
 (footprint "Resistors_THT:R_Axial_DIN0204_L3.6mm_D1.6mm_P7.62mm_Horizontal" (layer "F.Cu") (at 80.645 80.01 -90)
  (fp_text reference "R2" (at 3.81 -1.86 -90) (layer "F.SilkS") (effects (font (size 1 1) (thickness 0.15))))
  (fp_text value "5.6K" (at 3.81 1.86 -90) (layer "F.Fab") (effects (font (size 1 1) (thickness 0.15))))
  (fp_line (start 5.67 0.86) (end 5.67 -0.86) (layer "F.SilkS") (width 0.12))
  (fp_line (start 5.67 -0.86) (end 1.95 -0.86) (layer "F.SilkS") (width 0.12))
  (fp_line (start 6.74 0) (end 5.67 0) (layer "F.SilkS") (width 0.12))
  (fp_line (start 1.95 -0.86) (end 1.95 0.86) (layer "F.SilkS") (width 0.12))
  (fp_line (start 1.95 0.86) (end 5.67 0.86) (layer "F.SilkS") (width 0.12))
  (fp_line (start 0.88 0) (end 1.95 0) (layer "F.SilkS") (width 0.12))
  (pad "1" thru_hole circle locked (at 0 0 270) (size 2 2) (drill 0.8) (layers *.Cu *.Mask) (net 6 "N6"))
  (pad "2" thru_hole circle locked (at 7.62 0 270) (size 2 2) (drill 0.8) (layers *.Cu *.Mask) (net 2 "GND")))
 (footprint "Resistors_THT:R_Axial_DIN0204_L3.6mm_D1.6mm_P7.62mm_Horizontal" (layer "F.Cu") (at 78.105 87.63 90)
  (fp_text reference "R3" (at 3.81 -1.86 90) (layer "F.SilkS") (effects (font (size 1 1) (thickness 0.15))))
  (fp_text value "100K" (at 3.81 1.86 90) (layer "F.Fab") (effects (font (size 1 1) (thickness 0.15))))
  (fp_line (start 5.67 -0.86) (end 1.95 -0.86) (layer "F.SilkS") (width 0.12))
  (fp_line (start 6.74 0) (end 5.67 0) (layer "F.SilkS") (width 0.12))
  (fp_line (start 1.95 -0.86) (end 1.95 0.86) (layer "F.SilkS") (width 0.12))
  (fp_line (start 0.88 0) (end 1.95 0) (layer "F.SilkS") (width 0.12))
  (fp_line (start 5.67 0.86) (end 5.67 -0.86) (layer "F.SilkS") (width 0.12))
  (fp_line (start 1.95 0.86) (end 5.67 0.86) (layer "F.SilkS") (width 0.12))
  (pad "1" thru_hole circle locked (at 0 0 90) (size 2 2) (drill 0.8) (layers *.Cu *.Mask) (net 5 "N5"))
  (pad "2" thru_hole circle locked (at 7.62 0 90) (size 2 2) (drill 0.8) (layers *.Cu *.Mask) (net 6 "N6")))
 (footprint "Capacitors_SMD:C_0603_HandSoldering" (layer "B.Cu") (at 70.485 84.455 -90)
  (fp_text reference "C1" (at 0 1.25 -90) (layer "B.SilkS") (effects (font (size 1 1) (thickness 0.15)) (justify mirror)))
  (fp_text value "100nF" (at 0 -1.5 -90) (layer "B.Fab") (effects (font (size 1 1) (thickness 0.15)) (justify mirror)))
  (pad "1" smd rect locked (at -0.95 0 270) (size 1.2 0.75) (layers "B.Cu" "B.Paste" "B.Mask") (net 3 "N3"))
  (pad "2" smd rect locked (at 0.95 0 270) (size 1.2 0.75) (layers "B.Cu" "B.Paste" "B.Mask") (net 4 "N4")))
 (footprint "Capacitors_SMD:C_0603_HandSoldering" (layer "B.Cu") (at 78.105 84.455 90)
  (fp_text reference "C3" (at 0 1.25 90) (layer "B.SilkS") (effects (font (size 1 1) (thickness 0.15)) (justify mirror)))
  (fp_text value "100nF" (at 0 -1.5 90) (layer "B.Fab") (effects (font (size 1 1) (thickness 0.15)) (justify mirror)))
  (pad "1" smd rect locked (at -0.95 0 90) (size 1.2 0.75) (layers "B.Cu" "B.Paste" "B.Mask") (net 2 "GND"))
  (pad "2" smd rect locked (at 0.95 0 90) (size 1.2 0.75) (layers "B.Cu" "B.Paste" "B.Mask") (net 1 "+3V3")))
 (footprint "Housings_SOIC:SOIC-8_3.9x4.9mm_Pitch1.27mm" (layer "B.Cu") (at 74.295 84.455 90)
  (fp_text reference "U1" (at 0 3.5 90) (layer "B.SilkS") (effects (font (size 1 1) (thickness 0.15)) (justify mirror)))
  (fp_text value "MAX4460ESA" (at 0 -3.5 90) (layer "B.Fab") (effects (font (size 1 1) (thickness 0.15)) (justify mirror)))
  (pad "1" smd rect locked (at -2.7 1.905 90) (size 1.55 0.6) (layers "B.Cu" "B.Paste" "B.Mask") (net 5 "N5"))
  (pad "2" smd rect locked (at -2.7 0.635 90) (size 1.55 0.6) (layers "B.Cu" "B.Paste" "B.Mask") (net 2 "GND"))
  (pad "3" smd rect locked (at -2.7 -0.635 90) (size 1.55 0.6) (layers "B.Cu" "B.Paste" "B.Mask") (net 4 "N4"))
  (pad "4" smd rect locked (at -2.7 -1.905 90) (size 1.55 0.6) (layers "B.Cu" "B.Paste" "B.Mask"))
  (pad "5" smd rect locked (at 2.7 -1.905 90) (size 1.55 0.6) (layers "B.Cu" "B.Paste" "B.Mask"))
  (pad "6" smd rect locked (at 2.7 -0.635 90) (size 1.55 0.6) (layers "B.Cu" "B.Paste" "B.Mask") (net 3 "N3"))
  (pad "7" smd rect locked (at 2.7 0.635 90) (size 1.55 0.6) (layers "B.Cu" "B.Paste" "B.Mask") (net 1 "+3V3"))
  (pad "8" smd rect locked (at 2.7 1.905 90) (size 1.55 0.6) (layers "B.Cu" "B.Paste" "B.Mask") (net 6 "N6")))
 (gr_line (start 62.865 85.725) (end 61.595 86.995) (layer "Edge.Cuts") (width 0.15))
 (gr_line (start 61.595 72.39) (end 61.595 77.47) (layer "Edge.Cuts") (width 0.15))
 (gr_line (start 77.47 77.47) (end 72.39 72.39) (layer "Edge.Cuts") (width 0.15))
 (gr_line (start 83.185 79.375) (end 81.28 77.47) (layer "Edge.Cuts") (width 0.15))
 (gr_line (start 72.39 72.39) (end 61.595 72.39) (layer "Edge.Cuts") (width 0.15))
 (gr_line (start 62.865 78.74) (end 61.595 77.47) (layer "Edge.Cuts") (width 0.15))
 (gr_line (start 61.595 91.44) (end 83.185 91.44) (layer "Edge.Cuts") (width 0.15))
 (gr_line (start 81.28 77.47) (end 77.47 77.47) (layer "Edge.Cuts") (width 0.15))
 (gr_line (start 62.865 78.74) (end 62.865 85.725) (layer "Edge.Cuts") (width 0.15))
 (gr_line (start 83.185 91.44) (end 83.185 79.375) (layer "Edge.Cuts") (width 0.15))
 (gr_line (start 61.595 86.995) (end 61.595 91.44) (layer "Edge.Cuts") (width 0.15))
 (segment (start 69.545 82.565) (end 70.485 83.505) (width 0.8) (layer "B.Cu") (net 3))
 (segment (start 73.66 83.185) (end 73.34 83.505) (width 0.6) (layer "B.Cu") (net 3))
 (segment (start 73.34 83.505) (end 70.485 83.505) (width 0.6) (layer "B.Cu") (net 3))
 (segment (start 65.405 82.565) (end 68.58 82.565) (width 1) (layer "B.Cu") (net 3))
 (segment (start 68.58 82.565) (end 69.545 82.565) (width 0.8) (layer "B.Cu") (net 3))
 (segment (start 73.66 81.755) (end 73.66 83.185) (width 0.6) (layer "B.Cu") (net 3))
 (segment (start 69.825 86.065) (end 70.485 85.405) (width 0.8) (layer "B.Cu") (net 4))
 (segment (start 73.34 85.405) (end 73.66 85.725) (width 0.6) (layer "B.Cu") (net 4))
 (segment (start 73.66 85.725) (end 73.66 87.155) (width 0.6) (layer "B.Cu") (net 4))
 (segment (start 70.485 85.405) (end 73.34 85.405) (width 0.6) (layer "B.Cu") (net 4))
 (segment (start 65.405 86.065) (end 68.58 86.065) (width 1) (layer "B.Cu") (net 4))
 (segment (start 68.58 86.065) (end 69.825 86.065) (width 0.8) (layer "B.Cu") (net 4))
 (segment (start 75.25 85.405) (end 74.93 85.725) (width 0.8) (layer "B.Cu") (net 2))
 (segment (start 74.93 85.725) (end 74.93 87.155) (width 0.8) (layer "B.Cu") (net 2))
 (segment (start 64.46 79.065) (end 65.405 79.065) (width 1) (layer "B.Cu") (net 2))
 (segment (start 80.645 85.405) (end 80.645 85.725) (width 1) (layer "B.Cu") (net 2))
 (segment (start 80.645 85.725) (end 80.645 85.405) (width 1) (layer "B.Cu") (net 2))
 (segment (start 81.915 85.405) (end 80.645 85.405) (width 1) (layer "B.Cu") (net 2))
 (segment (start 82.55 84.77) (end 82.55 84.455) (width 1) (layer "B.Cu") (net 2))
 (segment (start 63.825 79.065) (end 62.23 77.47) (width 1) (layer "B.Cu") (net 2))
 (segment (start 77.47 78.105) (end 72.39 73.025) (width 1) (layer "B.Cu") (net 2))
 (segment (start 72.39 73.025) (end 62.23 73.025) (width 1) (layer "B.Cu") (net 2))
 (segment (start 81.28 78.105) (end 77.47 78.105) (width 1) (layer "B.Cu") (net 2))
 (segment (start 82.55 79.375) (end 82.55 84.455) (width 1) (layer "B.Cu") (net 2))
 (segment (start 68.58 79.065) (end 65.405 79.065) (width 1) (layer "B.Cu") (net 2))
 (segment (start 81.28 78.105) (end 82.55 79.375) (width 1) (layer "B.Cu") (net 2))
 (segment (start 78.105 85.405) (end 80.645 85.405) (width 1) (layer "B.Cu") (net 2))
 (segment (start 81.915 85.405) (end 82.55 84.77) (width 1) (layer "B.Cu") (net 2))
 (segment (start 62.23 73.025) (end 62.23 77.47) (width 1) (layer "B.Cu") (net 2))
 (segment (start 78.105 85.405) (end 75.25 85.405) (width 0.8) (layer "B.Cu") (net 2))
 (segment (start 80.645 87.63) (end 80.645 85.405) (width 1) (layer "B.Cu") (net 2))
 (segment (start 65.405 79.065) (end 63.825 79.065) (width 1) (layer "B.Cu") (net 2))
 (segment (start 72.39 75.565) (end 74.93 78.105) (width 0.8) (layer "B.Cu") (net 1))
 (segment (start 74.93 78.105) (end 74.93 81.755) (width 0.8) (layer "B.Cu") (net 1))
 (segment (start 75.245 83.505) (end 78.105 83.505) (width 0.8) (layer "B.Cu") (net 1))
 (segment (start 74.93 83.19) (end 75.245 83.505) (width 0.8) (layer "B.Cu") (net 1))
 (segment (start 68.58 75.565) (end 72.39 75.565) (width 0.8) (layer "B.Cu") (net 1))
 (segment (start 74.93 81.755) (end 74.93 83.19) (width 0.8) (layer "B.Cu") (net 1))
 (segment (start 68.58 75.565) (end 65.405 75.565) (width 1) (layer "B.Cu") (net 1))
 (segment (start 76.2 80.645) (end 76.835 80.01) (width 0.6) (layer "B.Cu") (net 6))
 (segment (start 76.835 80.01) (end 78.105 80.01) (width 0.6) (layer "B.Cu") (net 6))
 (segment (start 76.2 81.755) (end 76.2 80.645) (width 0.6) (layer "B.Cu") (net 6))
 (segment (start 78.105 80.01) (end 80.645 80.01) (width 0.8) (layer "B.Cu") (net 6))
 (segment (start 73.025 89.535) (end 72.39 90.17) (width 0.6) (layer "B.Cu") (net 5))
 (segment (start 76.2 89.535) (end 73.025 89.535) (width 0.6) (layer "B.Cu") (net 5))
 (segment (start 77.63 87.155) (end 76.2 87.155) (width 0.6) (layer "B.Cu") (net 5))
 (segment (start 76.2 87.155) (end 76.2 89.535) (width 0.6) (layer "B.Cu") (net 5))
 (segment (start 78.105 87.63) (end 77.63 87.155) (width 0.6) (layer "B.Cu") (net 5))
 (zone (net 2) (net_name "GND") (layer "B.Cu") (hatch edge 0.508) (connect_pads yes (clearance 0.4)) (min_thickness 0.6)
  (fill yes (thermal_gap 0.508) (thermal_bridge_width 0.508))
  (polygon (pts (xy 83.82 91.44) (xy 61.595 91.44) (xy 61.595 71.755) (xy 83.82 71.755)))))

